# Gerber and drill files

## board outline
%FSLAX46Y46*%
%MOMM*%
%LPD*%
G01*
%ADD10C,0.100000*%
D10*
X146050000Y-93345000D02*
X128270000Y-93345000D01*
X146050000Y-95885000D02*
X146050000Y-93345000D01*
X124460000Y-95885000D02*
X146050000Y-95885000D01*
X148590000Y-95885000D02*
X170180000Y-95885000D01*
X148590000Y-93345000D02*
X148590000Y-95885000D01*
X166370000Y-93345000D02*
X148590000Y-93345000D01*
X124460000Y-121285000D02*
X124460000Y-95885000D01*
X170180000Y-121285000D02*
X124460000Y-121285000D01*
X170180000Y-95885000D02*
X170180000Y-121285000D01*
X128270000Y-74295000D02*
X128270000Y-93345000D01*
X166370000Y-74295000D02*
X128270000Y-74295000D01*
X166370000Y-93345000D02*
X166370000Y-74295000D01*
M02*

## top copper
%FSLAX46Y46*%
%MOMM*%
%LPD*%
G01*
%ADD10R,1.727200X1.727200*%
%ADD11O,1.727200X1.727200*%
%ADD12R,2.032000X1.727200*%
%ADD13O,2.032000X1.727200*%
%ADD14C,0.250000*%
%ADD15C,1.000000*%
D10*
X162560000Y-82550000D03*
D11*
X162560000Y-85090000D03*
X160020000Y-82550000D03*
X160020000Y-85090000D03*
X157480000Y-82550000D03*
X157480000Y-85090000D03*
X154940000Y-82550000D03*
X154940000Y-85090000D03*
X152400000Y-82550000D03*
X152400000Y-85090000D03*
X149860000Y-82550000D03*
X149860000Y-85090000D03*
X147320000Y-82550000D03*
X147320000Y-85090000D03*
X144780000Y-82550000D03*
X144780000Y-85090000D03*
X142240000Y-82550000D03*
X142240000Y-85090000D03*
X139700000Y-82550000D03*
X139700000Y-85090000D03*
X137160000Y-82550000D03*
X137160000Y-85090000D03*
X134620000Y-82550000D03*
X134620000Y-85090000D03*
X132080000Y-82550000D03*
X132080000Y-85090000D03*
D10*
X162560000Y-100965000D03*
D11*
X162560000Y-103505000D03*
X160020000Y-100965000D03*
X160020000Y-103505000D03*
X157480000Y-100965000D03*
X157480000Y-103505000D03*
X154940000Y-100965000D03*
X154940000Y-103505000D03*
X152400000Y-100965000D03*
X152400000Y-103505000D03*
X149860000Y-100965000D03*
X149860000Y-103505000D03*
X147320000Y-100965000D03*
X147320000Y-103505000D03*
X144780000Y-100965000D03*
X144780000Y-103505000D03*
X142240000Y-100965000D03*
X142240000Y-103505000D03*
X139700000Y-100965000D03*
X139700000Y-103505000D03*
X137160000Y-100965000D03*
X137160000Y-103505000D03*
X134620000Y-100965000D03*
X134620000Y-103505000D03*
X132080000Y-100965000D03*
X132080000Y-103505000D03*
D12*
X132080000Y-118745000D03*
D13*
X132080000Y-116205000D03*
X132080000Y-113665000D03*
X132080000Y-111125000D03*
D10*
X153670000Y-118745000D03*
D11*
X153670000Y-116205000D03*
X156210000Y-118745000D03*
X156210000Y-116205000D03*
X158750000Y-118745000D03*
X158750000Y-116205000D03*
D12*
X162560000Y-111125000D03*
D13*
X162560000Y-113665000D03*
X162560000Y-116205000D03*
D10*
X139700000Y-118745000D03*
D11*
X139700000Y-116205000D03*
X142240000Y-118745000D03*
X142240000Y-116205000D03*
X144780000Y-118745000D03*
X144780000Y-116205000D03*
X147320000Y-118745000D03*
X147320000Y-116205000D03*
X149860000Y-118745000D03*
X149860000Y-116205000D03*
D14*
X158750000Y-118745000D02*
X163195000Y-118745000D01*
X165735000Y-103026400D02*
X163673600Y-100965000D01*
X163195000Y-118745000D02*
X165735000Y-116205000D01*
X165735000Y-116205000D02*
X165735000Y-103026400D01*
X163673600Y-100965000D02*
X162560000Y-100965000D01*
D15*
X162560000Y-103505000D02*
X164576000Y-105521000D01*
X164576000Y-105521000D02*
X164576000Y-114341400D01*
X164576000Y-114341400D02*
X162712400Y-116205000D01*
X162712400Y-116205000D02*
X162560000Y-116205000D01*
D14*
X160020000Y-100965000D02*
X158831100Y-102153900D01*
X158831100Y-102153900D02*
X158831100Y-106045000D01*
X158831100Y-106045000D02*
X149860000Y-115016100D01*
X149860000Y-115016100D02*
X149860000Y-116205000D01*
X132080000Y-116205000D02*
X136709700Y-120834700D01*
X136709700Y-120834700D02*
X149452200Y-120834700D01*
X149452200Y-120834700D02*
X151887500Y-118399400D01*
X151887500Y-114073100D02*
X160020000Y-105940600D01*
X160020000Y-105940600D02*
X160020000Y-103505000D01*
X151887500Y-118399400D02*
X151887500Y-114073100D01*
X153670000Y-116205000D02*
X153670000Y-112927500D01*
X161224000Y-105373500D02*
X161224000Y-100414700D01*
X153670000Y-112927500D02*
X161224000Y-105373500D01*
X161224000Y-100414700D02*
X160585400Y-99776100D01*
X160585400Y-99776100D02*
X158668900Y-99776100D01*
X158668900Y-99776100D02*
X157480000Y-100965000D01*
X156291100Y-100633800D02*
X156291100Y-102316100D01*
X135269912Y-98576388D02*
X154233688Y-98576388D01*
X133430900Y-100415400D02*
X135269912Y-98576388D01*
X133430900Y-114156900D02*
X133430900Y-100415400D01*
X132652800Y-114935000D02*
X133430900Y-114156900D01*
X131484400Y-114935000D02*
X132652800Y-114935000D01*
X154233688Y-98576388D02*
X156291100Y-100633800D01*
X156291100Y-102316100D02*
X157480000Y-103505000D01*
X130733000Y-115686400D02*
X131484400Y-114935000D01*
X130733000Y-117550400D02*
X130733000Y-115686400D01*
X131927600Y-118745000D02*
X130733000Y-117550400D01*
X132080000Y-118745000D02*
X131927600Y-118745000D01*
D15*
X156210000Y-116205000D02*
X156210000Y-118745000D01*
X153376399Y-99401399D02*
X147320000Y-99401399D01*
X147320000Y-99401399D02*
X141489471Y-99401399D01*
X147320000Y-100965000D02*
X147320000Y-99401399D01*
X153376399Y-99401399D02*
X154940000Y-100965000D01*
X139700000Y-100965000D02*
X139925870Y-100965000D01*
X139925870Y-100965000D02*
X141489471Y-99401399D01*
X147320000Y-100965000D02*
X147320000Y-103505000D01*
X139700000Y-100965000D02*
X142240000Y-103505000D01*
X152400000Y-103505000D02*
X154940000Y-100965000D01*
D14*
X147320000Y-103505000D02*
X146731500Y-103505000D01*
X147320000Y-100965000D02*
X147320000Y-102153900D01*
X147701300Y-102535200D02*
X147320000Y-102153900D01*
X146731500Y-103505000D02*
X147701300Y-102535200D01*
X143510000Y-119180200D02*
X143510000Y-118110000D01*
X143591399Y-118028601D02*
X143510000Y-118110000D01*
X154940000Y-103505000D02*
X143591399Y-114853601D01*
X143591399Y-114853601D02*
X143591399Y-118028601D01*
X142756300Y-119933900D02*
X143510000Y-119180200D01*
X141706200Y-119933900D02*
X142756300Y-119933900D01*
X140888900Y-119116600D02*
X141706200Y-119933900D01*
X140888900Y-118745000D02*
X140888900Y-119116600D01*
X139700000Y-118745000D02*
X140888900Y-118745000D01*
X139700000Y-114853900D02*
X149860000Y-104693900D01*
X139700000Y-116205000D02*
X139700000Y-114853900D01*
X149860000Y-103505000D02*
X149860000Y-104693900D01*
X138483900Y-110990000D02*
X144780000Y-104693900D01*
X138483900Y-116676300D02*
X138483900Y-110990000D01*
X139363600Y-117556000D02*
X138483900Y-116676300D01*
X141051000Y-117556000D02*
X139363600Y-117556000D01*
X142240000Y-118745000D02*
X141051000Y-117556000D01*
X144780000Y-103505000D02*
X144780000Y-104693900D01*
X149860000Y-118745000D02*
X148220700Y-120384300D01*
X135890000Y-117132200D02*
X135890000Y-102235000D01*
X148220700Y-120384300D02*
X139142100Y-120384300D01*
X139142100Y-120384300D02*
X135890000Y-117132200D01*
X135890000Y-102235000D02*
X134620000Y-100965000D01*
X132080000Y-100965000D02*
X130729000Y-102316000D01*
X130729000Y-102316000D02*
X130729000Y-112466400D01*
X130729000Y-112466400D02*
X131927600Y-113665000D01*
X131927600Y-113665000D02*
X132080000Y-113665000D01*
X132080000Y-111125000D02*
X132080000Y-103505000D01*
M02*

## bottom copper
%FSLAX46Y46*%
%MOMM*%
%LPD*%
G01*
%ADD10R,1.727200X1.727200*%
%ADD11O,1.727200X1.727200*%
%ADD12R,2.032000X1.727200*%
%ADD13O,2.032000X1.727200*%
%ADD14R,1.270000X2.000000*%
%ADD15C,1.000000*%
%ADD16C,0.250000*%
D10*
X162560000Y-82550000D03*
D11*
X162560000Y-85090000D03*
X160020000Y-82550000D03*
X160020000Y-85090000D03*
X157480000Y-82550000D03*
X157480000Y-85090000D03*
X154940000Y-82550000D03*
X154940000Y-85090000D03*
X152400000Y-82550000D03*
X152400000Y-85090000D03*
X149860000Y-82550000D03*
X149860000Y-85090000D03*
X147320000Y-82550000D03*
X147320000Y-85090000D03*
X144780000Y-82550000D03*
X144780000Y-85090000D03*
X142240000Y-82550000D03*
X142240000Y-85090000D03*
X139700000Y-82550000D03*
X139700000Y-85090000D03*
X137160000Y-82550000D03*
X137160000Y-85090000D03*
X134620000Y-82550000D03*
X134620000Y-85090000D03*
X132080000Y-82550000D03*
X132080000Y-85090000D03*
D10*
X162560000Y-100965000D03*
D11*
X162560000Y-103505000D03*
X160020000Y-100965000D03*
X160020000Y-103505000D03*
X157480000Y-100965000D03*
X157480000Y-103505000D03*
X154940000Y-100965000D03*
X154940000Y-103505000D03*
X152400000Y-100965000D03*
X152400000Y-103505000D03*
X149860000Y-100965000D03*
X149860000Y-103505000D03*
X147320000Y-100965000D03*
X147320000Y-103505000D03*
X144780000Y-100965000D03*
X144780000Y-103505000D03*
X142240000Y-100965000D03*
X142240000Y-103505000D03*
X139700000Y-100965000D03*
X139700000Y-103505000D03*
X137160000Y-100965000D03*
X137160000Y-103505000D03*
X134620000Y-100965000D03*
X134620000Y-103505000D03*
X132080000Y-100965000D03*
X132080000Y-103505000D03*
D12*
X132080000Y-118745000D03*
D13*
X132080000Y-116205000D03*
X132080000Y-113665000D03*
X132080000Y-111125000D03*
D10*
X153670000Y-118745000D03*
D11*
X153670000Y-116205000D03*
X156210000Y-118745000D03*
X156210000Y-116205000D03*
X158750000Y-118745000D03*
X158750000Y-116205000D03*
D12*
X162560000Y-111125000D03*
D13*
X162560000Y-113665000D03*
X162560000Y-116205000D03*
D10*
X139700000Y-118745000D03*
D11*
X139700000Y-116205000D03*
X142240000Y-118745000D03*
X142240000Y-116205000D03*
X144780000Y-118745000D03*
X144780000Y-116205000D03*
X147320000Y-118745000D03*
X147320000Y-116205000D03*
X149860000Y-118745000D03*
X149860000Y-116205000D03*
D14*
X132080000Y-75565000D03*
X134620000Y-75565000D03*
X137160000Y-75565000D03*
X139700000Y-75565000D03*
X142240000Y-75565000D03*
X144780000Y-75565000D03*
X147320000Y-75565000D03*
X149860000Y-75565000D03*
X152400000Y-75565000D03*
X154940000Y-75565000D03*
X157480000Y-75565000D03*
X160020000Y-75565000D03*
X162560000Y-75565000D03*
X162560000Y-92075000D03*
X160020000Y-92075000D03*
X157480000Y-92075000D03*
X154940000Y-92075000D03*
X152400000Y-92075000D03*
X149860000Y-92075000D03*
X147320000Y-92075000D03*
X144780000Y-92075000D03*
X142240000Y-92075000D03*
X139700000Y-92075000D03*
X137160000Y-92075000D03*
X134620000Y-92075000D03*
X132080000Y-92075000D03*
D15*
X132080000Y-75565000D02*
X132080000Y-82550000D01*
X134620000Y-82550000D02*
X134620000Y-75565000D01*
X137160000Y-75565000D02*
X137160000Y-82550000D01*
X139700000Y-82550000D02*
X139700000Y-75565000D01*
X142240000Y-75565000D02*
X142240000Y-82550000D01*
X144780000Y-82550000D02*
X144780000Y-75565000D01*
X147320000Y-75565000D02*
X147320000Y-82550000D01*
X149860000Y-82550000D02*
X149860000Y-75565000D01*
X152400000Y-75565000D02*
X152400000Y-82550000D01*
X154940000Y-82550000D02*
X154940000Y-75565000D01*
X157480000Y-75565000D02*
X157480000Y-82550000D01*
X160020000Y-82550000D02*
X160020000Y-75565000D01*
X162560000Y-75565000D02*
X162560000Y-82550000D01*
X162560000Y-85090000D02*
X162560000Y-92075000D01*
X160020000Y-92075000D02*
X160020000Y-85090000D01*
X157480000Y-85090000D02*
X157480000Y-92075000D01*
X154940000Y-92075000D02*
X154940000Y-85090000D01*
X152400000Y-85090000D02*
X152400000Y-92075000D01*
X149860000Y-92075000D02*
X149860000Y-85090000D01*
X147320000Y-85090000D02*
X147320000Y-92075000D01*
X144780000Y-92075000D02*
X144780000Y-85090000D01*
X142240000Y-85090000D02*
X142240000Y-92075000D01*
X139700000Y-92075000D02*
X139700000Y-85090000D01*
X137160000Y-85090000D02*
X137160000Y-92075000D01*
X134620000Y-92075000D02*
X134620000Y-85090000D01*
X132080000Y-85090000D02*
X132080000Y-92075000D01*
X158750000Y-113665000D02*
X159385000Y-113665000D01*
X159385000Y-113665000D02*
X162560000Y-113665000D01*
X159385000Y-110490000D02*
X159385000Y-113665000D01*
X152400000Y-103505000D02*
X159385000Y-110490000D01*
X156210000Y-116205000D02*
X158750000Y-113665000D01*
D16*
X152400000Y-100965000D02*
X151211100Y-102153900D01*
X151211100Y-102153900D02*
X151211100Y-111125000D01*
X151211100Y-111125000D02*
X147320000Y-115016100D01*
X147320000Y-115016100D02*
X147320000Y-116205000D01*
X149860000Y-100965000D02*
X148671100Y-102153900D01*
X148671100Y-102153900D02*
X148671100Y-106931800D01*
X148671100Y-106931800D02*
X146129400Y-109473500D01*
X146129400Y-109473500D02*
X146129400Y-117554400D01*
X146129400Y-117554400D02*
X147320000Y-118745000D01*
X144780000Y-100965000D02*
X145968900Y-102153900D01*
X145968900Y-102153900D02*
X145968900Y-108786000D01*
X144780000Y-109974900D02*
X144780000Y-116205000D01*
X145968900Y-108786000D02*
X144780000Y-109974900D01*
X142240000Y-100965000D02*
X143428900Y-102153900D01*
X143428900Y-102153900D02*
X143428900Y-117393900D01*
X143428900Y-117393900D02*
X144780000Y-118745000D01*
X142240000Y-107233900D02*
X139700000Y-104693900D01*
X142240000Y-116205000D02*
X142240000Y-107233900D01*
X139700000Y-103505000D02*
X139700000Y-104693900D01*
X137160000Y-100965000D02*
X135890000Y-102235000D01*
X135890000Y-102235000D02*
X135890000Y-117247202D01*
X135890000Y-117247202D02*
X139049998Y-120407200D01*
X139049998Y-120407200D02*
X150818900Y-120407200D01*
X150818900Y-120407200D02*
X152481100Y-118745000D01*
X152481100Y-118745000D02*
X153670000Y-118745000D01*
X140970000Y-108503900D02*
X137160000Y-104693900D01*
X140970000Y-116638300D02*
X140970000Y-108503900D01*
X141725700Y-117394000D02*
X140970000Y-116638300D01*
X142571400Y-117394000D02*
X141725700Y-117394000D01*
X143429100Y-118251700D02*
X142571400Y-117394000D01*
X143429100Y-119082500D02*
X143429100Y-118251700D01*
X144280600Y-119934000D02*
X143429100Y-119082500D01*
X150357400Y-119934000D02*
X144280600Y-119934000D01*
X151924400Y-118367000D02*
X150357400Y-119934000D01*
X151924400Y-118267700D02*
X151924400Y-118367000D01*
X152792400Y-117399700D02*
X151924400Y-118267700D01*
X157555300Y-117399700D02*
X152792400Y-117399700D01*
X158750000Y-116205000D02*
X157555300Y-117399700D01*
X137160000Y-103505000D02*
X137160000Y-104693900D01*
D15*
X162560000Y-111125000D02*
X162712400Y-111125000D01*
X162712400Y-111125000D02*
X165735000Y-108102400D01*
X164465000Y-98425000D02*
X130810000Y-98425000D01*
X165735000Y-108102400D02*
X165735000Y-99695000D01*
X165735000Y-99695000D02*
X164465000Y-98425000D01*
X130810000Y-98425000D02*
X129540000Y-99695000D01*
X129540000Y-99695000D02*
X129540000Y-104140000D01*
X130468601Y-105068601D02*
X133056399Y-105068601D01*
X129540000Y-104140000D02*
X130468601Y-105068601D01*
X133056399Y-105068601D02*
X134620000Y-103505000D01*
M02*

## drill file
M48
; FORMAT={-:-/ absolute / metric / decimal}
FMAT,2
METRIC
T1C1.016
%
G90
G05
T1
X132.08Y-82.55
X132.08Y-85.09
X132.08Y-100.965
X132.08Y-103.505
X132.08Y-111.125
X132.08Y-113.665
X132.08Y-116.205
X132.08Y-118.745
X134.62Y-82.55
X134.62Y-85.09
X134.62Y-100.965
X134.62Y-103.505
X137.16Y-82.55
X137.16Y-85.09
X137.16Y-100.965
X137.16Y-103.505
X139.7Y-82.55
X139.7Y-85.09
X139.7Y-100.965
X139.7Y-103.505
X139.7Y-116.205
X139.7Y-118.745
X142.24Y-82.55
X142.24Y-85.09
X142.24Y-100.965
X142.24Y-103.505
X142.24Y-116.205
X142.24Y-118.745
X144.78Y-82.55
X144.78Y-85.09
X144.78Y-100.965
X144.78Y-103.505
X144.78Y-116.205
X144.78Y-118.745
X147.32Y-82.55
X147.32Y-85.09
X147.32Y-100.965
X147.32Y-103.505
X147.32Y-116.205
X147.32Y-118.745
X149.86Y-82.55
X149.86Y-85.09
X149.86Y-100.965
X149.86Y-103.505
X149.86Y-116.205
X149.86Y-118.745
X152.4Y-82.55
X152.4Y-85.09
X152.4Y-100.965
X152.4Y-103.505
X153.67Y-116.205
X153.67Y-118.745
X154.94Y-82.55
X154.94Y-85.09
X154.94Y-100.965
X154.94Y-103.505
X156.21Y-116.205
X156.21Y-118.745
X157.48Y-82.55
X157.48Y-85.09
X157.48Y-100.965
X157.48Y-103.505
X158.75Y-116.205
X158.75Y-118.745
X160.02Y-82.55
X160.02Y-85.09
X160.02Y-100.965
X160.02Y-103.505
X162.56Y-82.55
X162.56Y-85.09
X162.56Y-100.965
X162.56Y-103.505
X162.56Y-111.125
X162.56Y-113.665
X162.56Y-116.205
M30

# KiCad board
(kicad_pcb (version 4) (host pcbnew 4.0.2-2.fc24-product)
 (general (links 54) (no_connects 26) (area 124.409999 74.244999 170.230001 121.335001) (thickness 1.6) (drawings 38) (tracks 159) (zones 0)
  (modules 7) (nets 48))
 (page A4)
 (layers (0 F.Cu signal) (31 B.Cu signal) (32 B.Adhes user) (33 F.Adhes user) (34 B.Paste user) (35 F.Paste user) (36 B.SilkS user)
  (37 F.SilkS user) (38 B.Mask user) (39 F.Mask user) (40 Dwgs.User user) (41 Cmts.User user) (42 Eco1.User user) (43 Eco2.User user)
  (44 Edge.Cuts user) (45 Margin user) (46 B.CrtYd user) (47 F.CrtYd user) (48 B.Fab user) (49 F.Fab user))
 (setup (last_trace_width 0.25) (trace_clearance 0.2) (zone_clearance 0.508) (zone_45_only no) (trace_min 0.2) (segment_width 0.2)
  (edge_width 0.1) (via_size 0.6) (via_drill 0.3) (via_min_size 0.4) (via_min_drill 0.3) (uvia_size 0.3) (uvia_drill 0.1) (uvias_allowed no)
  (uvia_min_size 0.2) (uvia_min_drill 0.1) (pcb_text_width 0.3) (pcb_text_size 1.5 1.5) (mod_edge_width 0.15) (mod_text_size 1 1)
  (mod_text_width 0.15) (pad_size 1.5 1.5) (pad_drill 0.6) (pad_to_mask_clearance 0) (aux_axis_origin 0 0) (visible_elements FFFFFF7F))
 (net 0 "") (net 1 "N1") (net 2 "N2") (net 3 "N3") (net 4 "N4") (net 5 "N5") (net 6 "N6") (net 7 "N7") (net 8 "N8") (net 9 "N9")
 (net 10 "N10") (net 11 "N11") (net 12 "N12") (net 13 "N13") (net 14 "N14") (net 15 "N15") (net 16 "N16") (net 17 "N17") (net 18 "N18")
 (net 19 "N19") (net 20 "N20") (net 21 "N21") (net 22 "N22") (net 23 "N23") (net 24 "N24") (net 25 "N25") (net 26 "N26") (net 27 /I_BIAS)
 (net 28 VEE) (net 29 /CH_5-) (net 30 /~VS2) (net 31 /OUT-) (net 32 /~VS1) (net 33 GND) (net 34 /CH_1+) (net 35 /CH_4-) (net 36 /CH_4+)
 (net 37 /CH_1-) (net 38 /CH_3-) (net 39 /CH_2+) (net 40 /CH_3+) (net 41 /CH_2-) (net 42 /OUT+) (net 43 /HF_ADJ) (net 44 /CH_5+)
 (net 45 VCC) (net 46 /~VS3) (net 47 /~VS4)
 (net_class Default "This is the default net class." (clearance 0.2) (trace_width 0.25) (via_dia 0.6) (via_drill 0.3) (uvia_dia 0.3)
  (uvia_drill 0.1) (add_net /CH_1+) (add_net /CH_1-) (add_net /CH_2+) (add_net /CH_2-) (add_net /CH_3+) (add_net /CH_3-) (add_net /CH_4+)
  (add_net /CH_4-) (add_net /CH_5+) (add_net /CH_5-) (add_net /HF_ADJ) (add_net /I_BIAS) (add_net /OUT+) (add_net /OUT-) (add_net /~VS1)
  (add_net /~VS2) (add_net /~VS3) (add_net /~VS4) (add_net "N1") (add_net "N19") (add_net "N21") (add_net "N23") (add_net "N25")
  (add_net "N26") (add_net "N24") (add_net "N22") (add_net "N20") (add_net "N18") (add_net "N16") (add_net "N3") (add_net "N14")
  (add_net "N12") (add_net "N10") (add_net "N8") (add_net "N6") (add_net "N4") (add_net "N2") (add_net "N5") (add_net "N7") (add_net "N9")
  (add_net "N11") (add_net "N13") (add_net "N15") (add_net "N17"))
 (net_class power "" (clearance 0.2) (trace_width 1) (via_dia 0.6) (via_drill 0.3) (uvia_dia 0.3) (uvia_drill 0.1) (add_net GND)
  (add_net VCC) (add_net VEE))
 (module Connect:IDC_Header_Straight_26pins (layer F.Cu) (at 162.56 82.55 180)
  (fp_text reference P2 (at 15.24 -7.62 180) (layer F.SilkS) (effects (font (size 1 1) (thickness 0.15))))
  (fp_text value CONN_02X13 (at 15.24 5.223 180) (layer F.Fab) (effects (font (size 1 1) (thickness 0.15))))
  (pad 1 thru_hole rect (at 0 0 180) (size 1.7272 1.7272) (drill 1.016) (layers *.Cu *.Mask F.SilkS) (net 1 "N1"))
  (pad 2 thru_hole oval (at 0 -2.54 180) (size 1.7272 1.7272) (drill 1.016) (layers *.Cu *.Mask F.SilkS) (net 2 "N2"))
  (pad 3 thru_hole oval (at 2.54 0 180) (size 1.7272 1.7272) (drill 1.016) (layers *.Cu *.Mask F.SilkS) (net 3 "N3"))
  (pad 4 thru_hole oval (at 2.54 -2.54 180) (size 1.7272 1.7272) (drill 1.016) (layers *.Cu *.Mask F.SilkS) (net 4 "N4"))
  (pad 5 thru_hole oval (at 5.08 0 180) (size 1.7272 1.7272) (drill 1.016) (layers *.Cu *.Mask F.SilkS) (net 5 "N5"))
  (pad 6 thru_hole oval (at 5.08 -2.54 180) (size 1.7272 1.7272) (drill 1.016) (layers *.Cu *.Mask F.SilkS) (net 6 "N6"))
  (pad 7 thru_hole oval (at 7.62 0 180) (size 1.7272 1.7272) (drill 1.016) (layers *.Cu *.Mask F.SilkS) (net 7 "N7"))
  (pad 8 thru_hole oval (at 7.62 -2.54 180) (size 1.7272 1.7272) (drill 1.016) (layers *.Cu *.Mask F.SilkS) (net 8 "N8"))
  (pad 9 thru_hole oval (at 10.16 0 180) (size 1.7272 1.7272) (drill 1.016) (layers *.Cu *.Mask F.SilkS) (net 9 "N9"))
  (pad 10 thru_hole oval (at 10.16 -2.54 180) (size 1.7272 1.7272) (drill 1.016) (layers *.Cu *.Mask F.SilkS) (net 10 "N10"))
  (pad 11 thru_hole oval (at 12.7 0 180) (size 1.7272 1.7272) (drill 1.016) (layers *.Cu *.Mask F.SilkS) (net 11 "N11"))
  (pad 12 thru_hole oval (at 12.7 -2.54 180) (size 1.7272 1.7272) (drill 1.016) (layers *.Cu *.Mask F.SilkS) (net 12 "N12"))
  (pad 13 thru_hole oval (at 15.24 0 180) (size 1.7272 1.7272) (drill 1.016) (layers *.Cu *.Mask F.SilkS) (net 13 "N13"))
  (pad 14 thru_hole oval (at 15.24 -2.54 180) (size 1.7272 1.7272) (drill 1.016) (layers *.Cu *.Mask F.SilkS) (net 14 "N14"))
  (pad 15 thru_hole oval (at 17.78 0 180) (size 1.7272 1.7272) (drill 1.016) (layers *.Cu *.Mask F.SilkS) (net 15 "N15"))
  (pad 16 thru_hole oval (at 17.78 -2.54 180) (size 1.7272 1.7272) (drill 1.016) (layers *.Cu *.Mask F.SilkS) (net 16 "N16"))
  (pad 17 thru_hole oval (at 20.32 0 180) (size 1.7272 1.7272) (drill 1.016) (layers *.Cu *.Mask F.SilkS) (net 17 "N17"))
  (pad 18 thru_hole oval (at 20.32 -2.54 180) (size 1.7272 1.7272) (drill 1.016) (layers *.Cu *.Mask F.SilkS) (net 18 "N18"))
  (pad 19 thru_hole oval (at 22.86 0 180) (size 1.7272 1.7272) (drill 1.016) (layers *.Cu *.Mask F.SilkS) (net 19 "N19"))
  (pad 20 thru_hole oval (at 22.86 -2.54 180) (size 1.7272 1.7272) (drill 1.016) (layers *.Cu *.Mask F.SilkS) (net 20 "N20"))
  (pad 21 thru_hole oval (at 25.4 0 180) (size 1.7272 1.7272) (drill 1.016) (layers *.Cu *.Mask F.SilkS) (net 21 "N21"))
  (pad 22 thru_hole oval (at 25.4 -2.54 180) (size 1.7272 1.7272) (drill 1.016) (layers *.Cu *.Mask F.SilkS) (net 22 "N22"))
  (pad 23 thru_hole oval (at 27.94 0 180) (size 1.7272 1.7272) (drill 1.016) (layers *.Cu *.Mask F.SilkS) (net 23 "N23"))
  (pad 24 thru_hole oval (at 27.94 -2.54 180) (size 1.7272 1.7272) (drill 1.016) (layers *.Cu *.Mask F.SilkS) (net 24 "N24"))
  (pad 25 thru_hole oval (at 30.48 0 180) (size 1.7272 1.7272) (drill 1.016) (layers *.Cu *.Mask F.SilkS) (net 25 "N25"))
  (pad 26 thru_hole oval (at 30.48 -2.54 180) (size 1.7272 1.7272) (drill 1.016) (layers *.Cu *.Mask F.SilkS) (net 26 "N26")))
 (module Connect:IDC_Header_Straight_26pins (layer F.Cu) (at 162.56 100.965 180)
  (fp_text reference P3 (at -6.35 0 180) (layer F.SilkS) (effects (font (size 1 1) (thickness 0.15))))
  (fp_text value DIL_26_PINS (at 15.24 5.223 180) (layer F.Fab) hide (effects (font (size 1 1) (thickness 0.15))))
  (pad 1 thru_hole rect (at 0 0 180) (size 1.7272 1.7272) (drill 1.016) (layers *.Cu *.Mask F.SilkS) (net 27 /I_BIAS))
  (pad 2 thru_hole oval (at 0 -2.54 180) (size 1.7272 1.7272) (drill 1.016) (layers *.Cu *.Mask F.SilkS) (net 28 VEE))
  (pad 3 thru_hole oval (at 2.54 0 180) (size 1.7272 1.7272) (drill 1.016) (layers *.Cu *.Mask F.SilkS) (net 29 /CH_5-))
  (pad 4 thru_hole oval (at 2.54 -2.54 180) (size 1.7272 1.7272) (drill 1.016) (layers *.Cu *.Mask F.SilkS) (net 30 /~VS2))
  (pad 5 thru_hole oval (at 5.08 0 180) (size 1.7272 1.7272) (drill 1.016) (layers *.Cu *.Mask F.SilkS) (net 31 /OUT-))
  (pad 6 thru_hole oval (at 5.08 -2.54 180) (size 1.7272 1.7272) (drill 1.016) (layers *.Cu *.Mask F.SilkS) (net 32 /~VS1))
  (pad 7 thru_hole oval (at 7.62 0 180) (size 1.7272 1.7272) (drill 1.016) (layers *.Cu *.Mask F.SilkS) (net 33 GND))
  (pad 8 thru_hole oval (at 7.62 -2.54 180) (size 1.7272 1.7272) (drill 1.016) (layers *.Cu *.Mask F.SilkS) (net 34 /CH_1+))
  (pad 9 thru_hole oval (at 10.16 0 180) (size 1.7272 1.7272) (drill 1.016) (layers *.Cu *.Mask F.SilkS) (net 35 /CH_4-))
  (pad 10 thru_hole oval (at 10.16 -2.54 180) (size 1.7272 1.7272) (drill 1.016) (layers *.Cu *.Mask F.SilkS) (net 33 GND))
  (pad 11 thru_hole oval (at 12.7 0 180) (size 1.7272 1.7272) (drill 1.016) (layers *.Cu *.Mask F.SilkS) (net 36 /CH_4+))
  (pad 12 thru_hole oval (at 12.7 -2.54 180) (size 1.7272 1.7272) (drill 1.016) (layers *.Cu *.Mask F.SilkS) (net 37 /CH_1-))
  (pad 13 thru_hole oval (at 15.24 0 180) (size 1.7272 1.7272) (drill 1.016) (layers *.Cu *.Mask F.SilkS) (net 33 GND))
  (pad 14 thru_hole oval (at 15.24 -2.54 180) (size 1.7272 1.7272) (drill 1.016) (layers *.Cu *.Mask F.SilkS) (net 33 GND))
  (pad 15 thru_hole oval (at 17.78 0 180) (size 1.7272 1.7272) (drill 1.016) (layers *.Cu *.Mask F.SilkS) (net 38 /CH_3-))
  (pad 16 thru_hole oval (at 17.78 -2.54 180) (size 1.7272 1.7272) (drill 1.016) (layers *.Cu *.Mask F.SilkS) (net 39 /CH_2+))
  (pad 17 thru_hole oval (at 20.32 0 180) (size 1.7272 1.7272) (drill 1.016) (layers *.Cu *.Mask F.SilkS) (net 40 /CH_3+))
  (pad 18 thru_hole oval (at 20.32 -2.54 180) (size 1.7272 1.7272) (drill 1.016) (layers *.Cu *.Mask F.SilkS) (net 33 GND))
  (pad 19 thru_hole oval (at 22.86 0 180) (size 1.7272 1.7272) (drill 1.016) (layers *.Cu *.Mask F.SilkS) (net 33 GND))
  (pad 20 thru_hole oval (at 22.86 -2.54 180) (size 1.7272 1.7272) (drill 1.016) (layers *.Cu *.Mask F.SilkS) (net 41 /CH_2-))
  (pad 21 thru_hole oval (at 25.4 0 180) (size 1.7272 1.7272) (drill 1.016) (layers *.Cu *.Mask F.SilkS) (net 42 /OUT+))
  (pad 22 thru_hole oval (at 25.4 -2.54 180) (size 1.7272 1.7272) (drill 1.016) (layers *.Cu *.Mask F.SilkS) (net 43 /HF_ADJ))
  (pad 23 thru_hole oval (at 27.94 0 180) (size 1.7272 1.7272) (drill 1.016) (layers *.Cu *.Mask F.SilkS) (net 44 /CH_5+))
  (pad 24 thru_hole oval (at 27.94 -2.54 180) (size 1.7272 1.7272) (drill 1.016) (layers *.Cu *.Mask F.SilkS) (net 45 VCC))
  (pad 25 thru_hole oval (at 30.48 0 180) (size 1.7272 1.7272) (drill 1.016) (layers *.Cu *.Mask F.SilkS) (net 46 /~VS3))
  (pad 26 thru_hole oval (at 30.48 -2.54 180) (size 1.7272 1.7272) (drill 1.016) (layers *.Cu *.Mask F.SilkS) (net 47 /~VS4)))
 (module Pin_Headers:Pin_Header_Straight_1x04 (layer F.Cu) (at 132.08 118.745 180)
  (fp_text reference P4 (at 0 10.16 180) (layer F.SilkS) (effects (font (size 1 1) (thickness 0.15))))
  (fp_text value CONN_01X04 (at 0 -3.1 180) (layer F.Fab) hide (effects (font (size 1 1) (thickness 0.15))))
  (pad 1 thru_hole rect (at 0 0 180) (size 2.032 1.7272) (drill 1.016) (layers *.Cu *.Mask F.SilkS) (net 32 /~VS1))
  (pad 2 thru_hole oval (at 0 2.54 180) (size 2.032 1.7272) (drill 1.016) (layers *.Cu *.Mask F.SilkS) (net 30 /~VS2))
  (pad 3 thru_hole oval (at 0 5.08 180) (size 2.032 1.7272) (drill 1.016) (layers *.Cu *.Mask F.SilkS) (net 46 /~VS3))
  (pad 4 thru_hole oval (at 0 7.62 180) (size 2.032 1.7272) (drill 1.016) (layers *.Cu *.Mask F.SilkS) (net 47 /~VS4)))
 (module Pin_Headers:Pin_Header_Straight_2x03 (layer F.Cu) (at 153.67 118.745 90)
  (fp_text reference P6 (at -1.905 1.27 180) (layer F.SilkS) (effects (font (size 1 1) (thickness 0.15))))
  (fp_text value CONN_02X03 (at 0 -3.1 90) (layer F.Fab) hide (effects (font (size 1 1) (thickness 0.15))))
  (pad 1 thru_hole rect (at 0 0 90) (size 1.7272 1.7272) (drill 1.016) (layers *.Cu *.Mask F.SilkS) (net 42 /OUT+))
  (pad 2 thru_hole oval (at 2.54 0 90) (size 1.7272 1.7272) (drill 1.016) (layers *.Cu *.Mask F.SilkS) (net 31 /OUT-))
  (pad 3 thru_hole oval (at 0 2.54 90) (size 1.7272 1.7272) (drill 1.016) (layers *.Cu *.Mask F.SilkS) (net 33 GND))
  (pad 4 thru_hole oval (at 2.54 2.54 90) (size 1.7272 1.7272) (drill 1.016) (layers *.Cu *.Mask F.SilkS) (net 33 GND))
  (pad 5 thru_hole oval (at 0 5.08 90) (size 1.7272 1.7272) (drill 1.016) (layers *.Cu *.Mask F.SilkS) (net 27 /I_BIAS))
  (pad 6 thru_hole oval (at 2.54 5.08 90) (size 1.7272 1.7272) (drill 1.016) (layers *.Cu *.Mask F.SilkS) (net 43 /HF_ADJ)))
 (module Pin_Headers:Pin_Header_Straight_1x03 (layer F.Cu) (at 162.56 111.125)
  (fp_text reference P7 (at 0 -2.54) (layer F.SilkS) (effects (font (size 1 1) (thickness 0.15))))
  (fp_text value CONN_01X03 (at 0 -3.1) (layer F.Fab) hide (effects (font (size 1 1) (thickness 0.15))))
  (pad 1 thru_hole rect (at 0 0) (size 2.032 1.7272) (drill 1.016) (layers *.Cu *.Mask F.SilkS) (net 45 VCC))
  (pad 2 thru_hole oval (at 0 2.54) (size 2.032 1.7272) (drill 1.016) (layers *.Cu *.Mask F.SilkS) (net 33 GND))
  (pad 3 thru_hole oval (at 0 5.08) (size 2.032 1.7272) (drill 1.016) (layers *.Cu *.Mask F.SilkS) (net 28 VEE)))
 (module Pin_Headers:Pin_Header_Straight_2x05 (layer F.Cu) (at 139.7 118.745 90)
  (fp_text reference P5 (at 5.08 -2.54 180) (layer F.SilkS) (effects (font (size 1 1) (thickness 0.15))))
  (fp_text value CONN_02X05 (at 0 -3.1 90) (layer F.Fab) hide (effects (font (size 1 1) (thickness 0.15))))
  (pad 1 thru_hole rect (at 0 0 90) (size 1.7272 1.7272) (drill 1.016) (layers *.Cu *.Mask F.SilkS) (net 34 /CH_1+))
  (pad 2 thru_hole oval (at 2.54 0 90) (size 1.7272 1.7272) (drill 1.016) (layers *.Cu *.Mask F.SilkS) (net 37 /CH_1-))
  (pad 3 thru_hole oval (at 0 2.54 90) (size 1.7272 1.7272) (drill 1.016) (layers *.Cu *.Mask F.SilkS) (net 39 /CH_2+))
  (pad 4 thru_hole oval (at 2.54 2.54 90) (size 1.7272 1.7272) (drill 1.016) (layers *.Cu *.Mask F.SilkS) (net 41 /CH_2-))
  (pad 5 thru_hole oval (at 0 5.08 90) (size 1.7272 1.7272) (drill 1.016) (layers *.Cu *.Mask F.SilkS) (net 40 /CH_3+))
  (pad 6 thru_hole oval (at 2.54 5.08 90) (size 1.7272 1.7272) (drill 1.016) (layers *.Cu *.Mask F.SilkS) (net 38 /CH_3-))
  (pad 7 thru_hole oval (at 0 7.62 90) (size 1.7272 1.7272) (drill 1.016) (layers *.Cu *.Mask F.SilkS) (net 36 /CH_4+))
  (pad 8 thru_hole oval (at 2.54 7.62 90) (size 1.7272 1.7272) (drill 1.016) (layers *.Cu *.Mask F.SilkS) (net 35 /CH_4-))
  (pad 9 thru_hole oval (at 0 10.16 90) (size 1.7272 1.7272) (drill 1.016) (layers *.Cu *.Mask F.SilkS) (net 44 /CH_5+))
  (pad 10 thru_hole oval (at 2.54 10.16 90) (size 1.7272 1.7272) (drill 1.016) (layers *.Cu *.Mask F.SilkS) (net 29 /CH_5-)))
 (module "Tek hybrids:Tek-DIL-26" (layer F.Cu) (at 128.27 74.295)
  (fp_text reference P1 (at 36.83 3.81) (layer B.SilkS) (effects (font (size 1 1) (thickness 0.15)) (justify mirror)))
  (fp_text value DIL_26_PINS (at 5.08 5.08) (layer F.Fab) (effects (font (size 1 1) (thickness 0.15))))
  (pad 13 connect rect (at 3.81 1.27) (size 1.27 2) (layers B.Cu B.Mask) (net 25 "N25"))
  (pad 12 connect rect (at 6.35 1.27) (size 1.27 2) (layers B.Cu B.Mask) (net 23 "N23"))
  (pad 11 connect rect (at 8.89 1.27) (size 1.27 2) (layers B.Cu B.Mask) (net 21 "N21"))
  (pad 10 connect rect (at 11.43 1.27) (size 1.27 2) (layers B.Cu B.Mask) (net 19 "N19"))
  (pad 9 connect rect (at 13.97 1.27) (size 1.27 2) (layers B.Cu B.Mask) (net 17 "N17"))
  (pad 8 connect rect (at 16.51 1.27) (size 1.27 2) (layers B.Cu B.Mask) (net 15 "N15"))
  (pad 7 connect rect (at 19.05 1.27) (size 1.27 2) (layers B.Cu B.Mask) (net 13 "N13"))
  (pad 6 connect rect (at 21.59 1.27) (size 1.27 2) (layers B.Cu B.Mask) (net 11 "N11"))
  (pad 5 connect rect (at 24.13 1.27) (size 1.27 2) (layers B.Cu B.Mask) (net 9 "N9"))
  (pad 4 connect rect (at 26.67 1.27) (size 1.27 2) (layers B.Cu B.Mask) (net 7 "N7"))
  (pad 3 connect rect (at 29.21 1.27) (size 1.27 2) (layers B.Cu B.Mask) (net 5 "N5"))
  (pad 2 connect rect (at 31.75 1.27) (size 1.27 2) (layers B.Cu B.Mask) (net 3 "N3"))
  (pad 1 connect rect (at 34.29 1.27) (size 1.27 2) (layers B.Cu B.Mask) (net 1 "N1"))
  (pad 26 connect rect (at 34.29 17.78) (size 1.27 2) (layers B.Cu B.Mask) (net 2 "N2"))
  (pad 25 connect rect (at 31.75 17.78) (size 1.27 2) (layers B.Cu B.Mask) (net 4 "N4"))
  (pad 24 connect rect (at 29.21 17.78) (size 1.27 2) (layers B.Cu B.Mask) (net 6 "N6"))
  (pad 23 connect rect (at 26.67 17.78) (size 1.27 2) (layers B.Cu B.Mask) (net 8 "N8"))
  (pad 22 connect rect (at 24.13 17.78) (size 1.27 2) (layers B.Cu B.Mask) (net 10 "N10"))
  (pad 21 connect rect (at 21.59 17.78) (size 1.27 2) (layers B.Cu B.Mask) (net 12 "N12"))
  (pad 20 connect rect (at 19.05 17.78) (size 1.27 2) (layers B.Cu B.Mask) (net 14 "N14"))
  (pad 19 connect rect (at 16.51 17.78) (size 1.27 2) (layers B.Cu B.Mask) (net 16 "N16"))
  (pad 18 connect rect (at 13.97 17.78) (size 1.27 2) (layers B.Cu B.Mask) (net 18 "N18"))
  (pad 17 connect rect (at 11.43 17.78) (size 1.27 2) (layers B.Cu B.Mask) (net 20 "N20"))
  (pad 16 connect rect (at 8.89 17.78) (size 1.27 2) (layers B.Cu B.Mask) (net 22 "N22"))
  (pad 15 connect rect (at 6.35 17.78) (size 1.27 2) (layers B.Cu B.Mask) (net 24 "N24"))
  (pad 14 connect rect (at 3.81 17.78) (size 1.27 2) (layers B.Cu B.Mask) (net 26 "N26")))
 (gr_line (start 146.05 93.345) (end 128.27 93.345) (layer Edge.Cuts) (width 0.1))
 (gr_line (start 146.05 95.885) (end 146.05 93.345) (layer Edge.Cuts) (width 0.1))
 (gr_line (start 124.46 95.885) (end 146.05 95.885) (layer Edge.Cuts) (width 0.1))
 (gr_line (start 148.59 95.885) (end 170.18 95.885) (layer Edge.Cuts) (width 0.1))
 (gr_line (start 148.59 93.345) (end 148.59 95.885) (layer Edge.Cuts) (width 0.1))
 (gr_line (start 166.37 93.345) (end 148.59 93.345) (layer Edge.Cuts) (width 0.1))
 (gr_line (start 124.46 121.285) (end 124.46 95.885) (layer Edge.Cuts) (width 0.1))
 (gr_line (start 170.18 121.285) (end 124.46 121.285) (layer Edge.Cuts) (width 0.1))
 (gr_line (start 170.18 95.885) (end 170.18 121.285) (layer Edge.Cuts) (width 0.1))
 (gr_line (start 128.27 74.295) (end 128.27 93.345) (layer Edge.Cuts) (width 0.1))
 (gr_line (start 166.37 74.295) (end 128.27 74.295) (layer Edge.Cuts) (width 0.1))
 (gr_line (start 166.37 93.345) (end 166.37 74.295) (layer Edge.Cuts) (width 0.1))
 (segment (start 132.08 75.565) (end 132.08 82.55) (width 1) (layer B.Cu) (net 25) (status 30))
 (segment (start 134.62 82.55) (end 134.62 75.565) (width 1) (layer B.Cu) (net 23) (status 30))
 (segment (start 137.16 75.565) (end 137.16 82.55) (width 1) (layer B.Cu) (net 21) (status 30))
 (segment (start 139.7 82.55) (end 139.7 75.565) (width 1) (layer B.Cu) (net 19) (status 30))
 (segment (start 142.24 75.565) (end 142.24 82.55) (width 1) (layer B.Cu) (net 17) (status 30))
 (segment (start 144.78 82.55) (end 144.78 75.565) (width 1) (layer B.Cu) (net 15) (status 30))
 (segment (start 147.32 75.565) (end 147.32 82.55) (width 1) (layer B.Cu) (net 13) (status 30))
 (segment (start 149.86 82.55) (end 149.86 75.565) (width 1) (layer B.Cu) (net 11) (status 30))
 (segment (start 152.4 75.565) (end 152.4 82.55) (width 1) (layer B.Cu) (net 9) (status 30))
 (segment (start 154.94 82.55) (end 154.94 75.565) (width 1) (layer B.Cu) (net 7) (status 30))
 (segment (start 157.48 75.565) (end 157.48 82.55) (width 1) (layer B.Cu) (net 5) (status 30))
 (segment (start 160.02 82.55) (end 160.02 75.565) (width 1) (layer B.Cu) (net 3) (status 30))
 (segment (start 162.56 75.565) (end 162.56 82.55) (width 1) (layer B.Cu) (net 1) (status 30))
 (segment (start 162.56 85.09) (end 162.56 92.075) (width 1) (layer B.Cu) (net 2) (status 30))
 (segment (start 160.02 92.075) (end 160.02 85.09) (width 1) (layer B.Cu) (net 4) (status 30))
 (segment (start 157.48 85.09) (end 157.48 92.075) (width 1) (layer B.Cu) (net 6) (status 30))
 (segment (start 154.94 92.075) (end 154.94 85.09) (width 1) (layer B.Cu) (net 8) (status 30))
 (segment (start 152.4 85.09) (end 152.4 92.075) (width 1) (layer B.Cu) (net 10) (status 30))
 (segment (start 149.86 92.075) (end 149.86 85.09) (width 1) (layer B.Cu) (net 12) (status 30))
 (segment (start 147.32 85.09) (end 147.32 92.075) (width 1) (layer B.Cu) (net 14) (status 30))
 (segment (start 144.78 92.075) (end 144.78 85.09) (width 1) (layer B.Cu) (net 16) (status 30))
 (segment (start 142.24 85.09) (end 142.24 92.075) (width 1) (layer B.Cu) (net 18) (status 30))
 (segment (start 139.7 92.075) (end 139.7 85.09) (width 1) (layer B.Cu) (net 20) (status 30))
 (segment (start 137.16 85.09) (end 137.16 92.075) (width 1) (layer B.Cu) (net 22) (status 30))
 (segment (start 134.62 92.075) (end 134.62 85.09) (width 1) (layer B.Cu) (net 24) (status 30))
 (segment (start 132.08 85.09) (end 132.08 92.075) (width 1) (layer B.Cu) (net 26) (status 30))
 (segment (start 158.75 118.745) (end 163.195 118.745) (width 0.25) (layer F.Cu) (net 27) (status 10))
 (segment (start 165.735 103.0264) (end 163.6736 100.965) (width 0.25) (layer F.Cu) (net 27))
 (segment (start 163.195 118.745) (end 165.735 116.205) (width 0.25) (layer F.Cu) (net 27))
 (segment (start 165.735 116.205) (end 165.735 103.0264) (width 0.25) (layer F.Cu) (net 27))
 (segment (start 163.6736 100.965) (end 162.56 100.965) (width 0.25) (layer F.Cu) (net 27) (status 20))
 (segment (start 162.56 103.505) (end 164.576 105.521) (width 1) (layer F.Cu) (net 28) (status 10))
 (segment (start 164.576 105.521) (end 164.576 114.3414) (width 1) (layer F.Cu) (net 28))
 (segment (start 164.576 114.3414) (end 162.7124 116.205) (width 1) (layer F.Cu) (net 28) (status 20))
 (segment (start 162.7124 116.205) (end 162.56 116.205) (width 1) (layer F.Cu) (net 28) (status 30))
 (segment (start 160.02 100.965) (end 158.8311 102.1539) (width 0.25) (layer F.Cu) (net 29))
 (segment (start 158.8311 102.1539) (end 158.8311 106.045) (width 0.25) (layer F.Cu) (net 29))
 (segment (start 158.8311 106.045) (end 149.86 115.0161) (width 0.25) (layer F.Cu) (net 29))
 (segment (start 149.86 115.0161) (end 149.86 116.205) (width 0.25) (layer F.Cu) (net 29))
 (segment (start 132.08 116.205) (end 136.7097 120.8347) (width 0.25) (layer F.Cu) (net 30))
 (segment (start 136.7097 120.8347) (end 149.4522 120.8347) (width 0.25) (layer F.Cu) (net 30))
 (segment (start 149.4522 120.8347) (end 151.8875 118.3994) (width 0.25) (layer F.Cu) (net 30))
 (segment (start 151.8875 114.0731) (end 160.02 105.9406) (width 0.25) (layer F.Cu) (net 30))
 (segment (start 160.02 105.9406) (end 160.02 103.505) (width 0.25) (layer F.Cu) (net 30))
 (segment (start 151.8875 118.3994) (end 151.8875 114.0731) (width 0.25) (layer F.Cu) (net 30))
 (segment (start 153.67 116.205) (end 153.67 112.9275) (width 0.25) (layer F.Cu) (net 31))
 (segment (start 161.224 105.3735) (end 161.224 100.4147) (width 0.25) (layer F.Cu) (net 31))
 (segment (start 153.67 112.9275) (end 161.224 105.3735) (width 0.25) (layer F.Cu) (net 31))
 (segment (start 161.224 100.4147) (end 160.5854 99.7761) (width 0.25) (layer F.Cu) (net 31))
 (segment (start 160.5854 99.7761) (end 158.6689 99.7761) (width 0.25) (layer F.Cu) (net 31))
 (segment (start 158.6689 99.7761) (end 157.48 100.965) (width 0.25) (layer F.Cu) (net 31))
 (segment (start 156.2911 100.6338) (end 156.2911 102.3161) (width 0.25) (layer F.Cu) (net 32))
 (segment (start 135.269912 98.576388) (end 154.233688 98.576388) (width 0.25) (layer F.Cu) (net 32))
 (segment (start 133.4309 100.4154) (end 135.269912 98.576388) (width 0.25) (layer F.Cu) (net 32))
 (segment (start 133.4309 114.1569) (end 133.4309 100.4154) (width 0.25) (layer F.Cu) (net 32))
 (segment (start 132.6528 114.935) (end 133.4309 114.1569) (width 0.25) (layer F.Cu) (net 32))
 (segment (start 131.4844 114.935) (end 132.6528 114.935) (width 0.25) (layer F.Cu) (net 32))
 (segment (start 154.233688 98.576388) (end 156.2911 100.6338) (width 0.25) (layer F.Cu) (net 32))
 (segment (start 156.2911 102.3161) (end 157.48 103.505) (width 0.25) (layer F.Cu) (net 32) (status 20))
 (segment (start 130.733 115.6864) (end 131.4844 114.935) (width 0.25) (layer F.Cu) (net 32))
 (segment (start 130.733 117.5504) (end 130.733 115.6864) (width 0.25) (layer F.Cu) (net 32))
 (segment (start 131.9276 118.745) (end 130.733 117.5504) (width 0.25) (layer F.Cu) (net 32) (status 10))
 (segment (start 132.08 118.745) (end 131.9276 118.745) (width 0.25) (layer F.Cu) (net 32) (status 30))
 (segment (start 156.21 116.205) (end 156.21 118.745) (width 1) (layer F.Cu) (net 33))
 (segment (start 153.376399 99.401399) (end 147.32 99.401399) (width 1) (layer F.Cu) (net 33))
 (segment (start 147.32 99.401399) (end 141.489471 99.401399) (width 1) (layer F.Cu) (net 33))
 (segment (start 147.32 100.965) (end 147.32 99.401399) (width 1) (layer F.Cu) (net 33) (status 10))
 (segment (start 153.376399 99.401399) (end 154.94 100.965) (width 1) (layer F.Cu) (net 33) (status 20))
 (segment (start 139.7 100.965) (end 139.92587 100.965) (width 1) (layer F.Cu) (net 33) (status 30))
 (segment (start 139.92587 100.965) (end 141.489471 99.401399) (width 1) (layer F.Cu) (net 33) (status 10))
 (segment (start 147.32 100.965) (end 147.32 103.505) (width 1) (layer F.Cu) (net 33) (status 30))
 (segment (start 139.7 100.965) (end 142.24 103.505) (width 1) (layer F.Cu) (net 33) (status 30))
 (segment (start 152.4 103.505) (end 154.94 100.965) (width 1) (layer F.Cu) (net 33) (status 30))
 (segment (start 158.75 113.665) (end 159.385 113.665) (width 1) (layer B.Cu) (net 33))
 (segment (start 159.385 113.665) (end 162.56 113.665) (width 1) (layer B.Cu) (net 33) (status 20))
 (segment (start 159.385 110.49) (end 159.385 113.665) (width 1) (layer B.Cu) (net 33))
 (segment (start 152.4 103.505) (end 159.385 110.49) (width 1) (layer B.Cu) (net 33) (status 10))
 (segment (start 156.21 116.205) (end 158.75 113.665) (width 1) (layer B.Cu) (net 33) (status 10))
 (segment (start 147.32 103.505) (end 146.7315 103.505) (width 0.25) (layer F.Cu) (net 33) (status 30))
 (segment (start 147.32 100.965) (end 147.32 102.1539) (width 0.25) (layer F.Cu) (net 33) (status 10))
 (segment (start 147.7013 102.5352) (end 147.32 102.1539) (width 0.25) (layer F.Cu) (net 33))
 (segment (start 146.7315 103.505) (end 147.7013 102.5352) (width 0.25) (layer F.Cu) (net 33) (status 10))
 (segment (start 143.51 119.1802) (end 143.51 118.11) (width 0.25) (layer F.Cu) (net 34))
 (segment (start 143.591399 118.028601) (end 143.51 118.11) (width 0.25) (layer F.Cu) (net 34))
 (segment (start 154.94 103.505) (end 143.591399 114.853601) (width 0.25) (layer F.Cu) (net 34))
 (segment (start 143.591399 114.853601) (end 143.591399 118.028601) (width 0.25) (layer F.Cu) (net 34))
 (segment (start 142.7563 119.9339) (end 143.51 119.1802) (width 0.25) (layer F.Cu) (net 34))
 (segment (start 141.7062 119.9339) (end 142.7563 119.9339) (width 0.25) (layer F.Cu) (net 34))
 (segment (start 140.8889 119.1166) (end 141.7062 119.9339) (width 0.25) (layer F.Cu) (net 34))
 (segment (start 140.8889 118.745) (end 140.8889 119.1166) (width 0.25) (layer F.Cu) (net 34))
 (segment (start 139.7 118.745) (end 140.8889 118.745) (width 0.25) (layer F.Cu) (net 34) (status 10))
 (segment (start 152.4 100.965) (end 151.2111 102.1539) (width 0.25) (layer B.Cu) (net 35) (status 10))
 (segment (start 151.2111 102.1539) (end 151.2111 111.125) (width 0.25) (layer B.Cu) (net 35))
 (segment (start 151.2111 111.125) (end 147.32 115.0161) (width 0.25) (layer B.Cu) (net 35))
 (segment (start 147.32 115.0161) (end 147.32 116.205) (width 0.25) (layer B.Cu) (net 35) (status 20))
 (segment (start 149.86 100.965) (end 148.6711 102.1539) (width 0.25) (layer B.Cu) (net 36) (status 10))
 (segment (start 148.6711 102.1539) (end 148.6711 106.9318) (width 0.25) (layer B.Cu) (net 36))
 (segment (start 148.6711 106.9318) (end 146.1294 109.4735) (width 0.25) (layer B.Cu) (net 36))
 (segment (start 146.1294 109.4735) (end 146.1294 117.5544) (width 0.25) (layer B.Cu) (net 36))
 (segment (start 146.1294 117.5544) (end 147.32 118.745) (width 0.25) (layer B.Cu) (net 36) (status 20))
 (segment (start 139.7 114.8539) (end 149.86 104.6939) (width 0.25) (layer F.Cu) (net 37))
 (segment (start 139.7 116.205) (end 139.7 114.8539) (width 0.25) (layer F.Cu) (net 37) (status 10))
 (segment (start 149.86 103.505) (end 149.86 104.6939) (width 0.25) (layer F.Cu) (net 37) (status 10))
 (segment (start 144.78 100.965) (end 145.9689 102.1539) (width 0.25) (layer B.Cu) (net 38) (status 10))
 (segment (start 145.9689 102.1539) (end 145.9689 108.786) (width 0.25) (layer B.Cu) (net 38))
 (segment (start 144.78 109.9749) (end 144.78 116.205) (width 0.25) (layer B.Cu) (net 38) (status 20))
 (segment (start 145.9689 108.786) (end 144.78 109.9749) (width 0.25) (layer B.Cu) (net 38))
 (segment (start 138.4839 110.99) (end 144.78 104.6939) (width 0.25) (layer F.Cu) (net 39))
 (segment (start 138.4839 116.6763) (end 138.4839 110.99) (width 0.25) (layer F.Cu) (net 39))
 (segment (start 139.3636 117.556) (end 138.4839 116.6763) (width 0.25) (layer F.Cu) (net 39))
 (segment (start 141.051 117.556) (end 139.3636 117.556) (width 0.25) (layer F.Cu) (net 39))
 (segment (start 142.24 118.745) (end 141.051 117.556) (width 0.25) (layer F.Cu) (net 39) (status 10))
 (segment (start 144.78 103.505) (end 144.78 104.6939) (width 0.25) (layer F.Cu) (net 39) (status 10))
 (segment (start 142.24 100.965) (end 143.4289 102.1539) (width 0.25) (layer B.Cu) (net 40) (status 10))
 (segment (start 143.4289 102.1539) (end 143.4289 117.3939) (width 0.25) (layer B.Cu) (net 40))
 (segment (start 143.4289 117.3939) (end 144.78 118.745) (width 0.25) (layer B.Cu) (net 40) (status 20))
 (segment (start 142.24 107.2339) (end 139.7 104.6939) (width 0.25) (layer B.Cu) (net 41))
 (segment (start 142.24 116.205) (end 142.24 107.2339) (width 0.25) (layer B.Cu) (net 41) (status 10))
 (segment (start 139.7 103.505) (end 139.7 104.6939) (width 0.25) (layer B.Cu) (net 41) (status 10))
 (segment (start 137.16 100.965) (end 135.89 102.235) (width 0.25) (layer B.Cu) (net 42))
 (segment (start 135.89 102.235) (end 135.89 117.247202) (width 0.25) (layer B.Cu) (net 42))
 (segment (start 135.89 117.247202) (end 139.049998 120.4072) (width 0.25) (layer B.Cu) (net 42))
 (segment (start 139.049998 120.4072) (end 150.8189 120.4072) (width 0.25) (layer B.Cu) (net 42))
 (segment (start 150.8189 120.4072) (end 152.4811 118.745) (width 0.25) (layer B.Cu) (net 42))
 (segment (start 152.4811 118.745) (end 153.67 118.745) (width 0.25) (layer B.Cu) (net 42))
 (segment (start 140.97 108.5039) (end 137.16 104.6939) (width 0.25) (layer B.Cu) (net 43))
 (segment (start 140.97 116.6383) (end 140.97 108.5039) (width 0.25) (layer B.Cu) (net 43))
 (segment (start 141.7257 117.394) (end 140.97 116.6383) (width 0.25) (layer B.Cu) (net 43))
 (segment (start 142.5714 117.394) (end 141.7257 117.394) (width 0.25) (layer B.Cu) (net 43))
 (segment (start 143.4291 118.2517) (end 142.5714 117.394) (width 0.25) (layer B.Cu) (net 43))
 (segment (start 143.4291 119.0825) (end 143.4291 118.2517) (width 0.25) (layer B.Cu) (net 43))
 (segment (start 144.2806 119.934) (end 143.4291 119.0825) (width 0.25) (layer B.Cu) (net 43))
 (segment (start 150.3574 119.934) (end 144.2806 119.934) (width 0.25) (layer B.Cu) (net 43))
 (segment (start 151.9244 118.367) (end 150.3574 119.934) (width 0.25) (layer B.Cu) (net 43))
 (segment (start 151.9244 118.2677) (end 151.9244 118.367) (width 0.25) (layer B.Cu) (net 43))
 (segment (start 152.7924 117.3997) (end 151.9244 118.2677) (width 0.25) (layer B.Cu) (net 43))
 (segment (start 157.5553 117.3997) (end 152.7924 117.3997) (width 0.25) (layer B.Cu) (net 43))
 (segment (start 158.75 116.205) (end 157.5553 117.3997) (width 0.25) (layer B.Cu) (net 43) (status 10))
 (segment (start 137.16 103.505) (end 137.16 104.6939) (width 0.25) (layer B.Cu) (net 43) (status 10))
 (segment (start 149.86 118.745) (end 148.2207 120.3843) (width 0.25) (layer F.Cu) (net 44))
 (segment (start 135.89 117.1322) (end 135.89 102.235) (width 0.25) (layer F.Cu) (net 44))
 (segment (start 148.2207 120.3843) (end 139.1421 120.3843) (width 0.25) (layer F.Cu) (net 44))
 (segment (start 139.1421 120.3843) (end 135.89 117.1322) (width 0.25) (layer F.Cu) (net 44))
 (segment (start 135.89 102.235) (end 134.62 100.965) (width 0.25) (layer F.Cu) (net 44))
 (segment (start 162.56 111.125) (end 162.7124 111.125) (width 1) (layer B.Cu) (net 45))
 (segment (start 162.7124 111.125) (end 165.735 108.1024) (width 1) (layer B.Cu) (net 45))
 (segment (start 164.465 98.425) (end 130.81 98.425) (width 1) (layer B.Cu) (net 45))
 (segment (start 165.735 108.1024) (end 165.735 99.695) (width 1) (layer B.Cu) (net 45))
 (segment (start 165.735 99.695) (end 164.465 98.425) (width 1) (layer B.Cu) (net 45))
 (segment (start 130.81 98.425) (end 129.54 99.695) (width 1) (layer B.Cu) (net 45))
 (segment (start 129.54 99.695) (end 129.54 104.14) (width 1) (layer B.Cu) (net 45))
 (segment (start 130.468601 105.068601) (end 133.056399 105.068601) (width 1) (layer B.Cu) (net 45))
 (segment (start 129.54 104.14) (end 130.468601 105.068601) (width 1) (layer B.Cu) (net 45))
 (segment (start 133.056399 105.068601) (end 134.62 103.505) (width 1) (layer B.Cu) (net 45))
 (segment (start 132.08 100.965) (end 130.729 102.316) (width 0.25) (layer F.Cu) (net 46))
 (segment (start 130.729 102.316) (end 130.729 112.4664) (width 0.25) (layer F.Cu) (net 46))
 (segment (start 130.729 112.4664) (end 131.9276 113.665) (width 0.25) (layer F.Cu) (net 46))
 (segment (start 131.9276 113.665) (end 132.08 113.665) (width 0.25) (layer F.Cu) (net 46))
 (segment (start 132.08 111.125) (end 132.08 103.505) (width 0.25) (layer F.Cu) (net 47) (status 30)))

